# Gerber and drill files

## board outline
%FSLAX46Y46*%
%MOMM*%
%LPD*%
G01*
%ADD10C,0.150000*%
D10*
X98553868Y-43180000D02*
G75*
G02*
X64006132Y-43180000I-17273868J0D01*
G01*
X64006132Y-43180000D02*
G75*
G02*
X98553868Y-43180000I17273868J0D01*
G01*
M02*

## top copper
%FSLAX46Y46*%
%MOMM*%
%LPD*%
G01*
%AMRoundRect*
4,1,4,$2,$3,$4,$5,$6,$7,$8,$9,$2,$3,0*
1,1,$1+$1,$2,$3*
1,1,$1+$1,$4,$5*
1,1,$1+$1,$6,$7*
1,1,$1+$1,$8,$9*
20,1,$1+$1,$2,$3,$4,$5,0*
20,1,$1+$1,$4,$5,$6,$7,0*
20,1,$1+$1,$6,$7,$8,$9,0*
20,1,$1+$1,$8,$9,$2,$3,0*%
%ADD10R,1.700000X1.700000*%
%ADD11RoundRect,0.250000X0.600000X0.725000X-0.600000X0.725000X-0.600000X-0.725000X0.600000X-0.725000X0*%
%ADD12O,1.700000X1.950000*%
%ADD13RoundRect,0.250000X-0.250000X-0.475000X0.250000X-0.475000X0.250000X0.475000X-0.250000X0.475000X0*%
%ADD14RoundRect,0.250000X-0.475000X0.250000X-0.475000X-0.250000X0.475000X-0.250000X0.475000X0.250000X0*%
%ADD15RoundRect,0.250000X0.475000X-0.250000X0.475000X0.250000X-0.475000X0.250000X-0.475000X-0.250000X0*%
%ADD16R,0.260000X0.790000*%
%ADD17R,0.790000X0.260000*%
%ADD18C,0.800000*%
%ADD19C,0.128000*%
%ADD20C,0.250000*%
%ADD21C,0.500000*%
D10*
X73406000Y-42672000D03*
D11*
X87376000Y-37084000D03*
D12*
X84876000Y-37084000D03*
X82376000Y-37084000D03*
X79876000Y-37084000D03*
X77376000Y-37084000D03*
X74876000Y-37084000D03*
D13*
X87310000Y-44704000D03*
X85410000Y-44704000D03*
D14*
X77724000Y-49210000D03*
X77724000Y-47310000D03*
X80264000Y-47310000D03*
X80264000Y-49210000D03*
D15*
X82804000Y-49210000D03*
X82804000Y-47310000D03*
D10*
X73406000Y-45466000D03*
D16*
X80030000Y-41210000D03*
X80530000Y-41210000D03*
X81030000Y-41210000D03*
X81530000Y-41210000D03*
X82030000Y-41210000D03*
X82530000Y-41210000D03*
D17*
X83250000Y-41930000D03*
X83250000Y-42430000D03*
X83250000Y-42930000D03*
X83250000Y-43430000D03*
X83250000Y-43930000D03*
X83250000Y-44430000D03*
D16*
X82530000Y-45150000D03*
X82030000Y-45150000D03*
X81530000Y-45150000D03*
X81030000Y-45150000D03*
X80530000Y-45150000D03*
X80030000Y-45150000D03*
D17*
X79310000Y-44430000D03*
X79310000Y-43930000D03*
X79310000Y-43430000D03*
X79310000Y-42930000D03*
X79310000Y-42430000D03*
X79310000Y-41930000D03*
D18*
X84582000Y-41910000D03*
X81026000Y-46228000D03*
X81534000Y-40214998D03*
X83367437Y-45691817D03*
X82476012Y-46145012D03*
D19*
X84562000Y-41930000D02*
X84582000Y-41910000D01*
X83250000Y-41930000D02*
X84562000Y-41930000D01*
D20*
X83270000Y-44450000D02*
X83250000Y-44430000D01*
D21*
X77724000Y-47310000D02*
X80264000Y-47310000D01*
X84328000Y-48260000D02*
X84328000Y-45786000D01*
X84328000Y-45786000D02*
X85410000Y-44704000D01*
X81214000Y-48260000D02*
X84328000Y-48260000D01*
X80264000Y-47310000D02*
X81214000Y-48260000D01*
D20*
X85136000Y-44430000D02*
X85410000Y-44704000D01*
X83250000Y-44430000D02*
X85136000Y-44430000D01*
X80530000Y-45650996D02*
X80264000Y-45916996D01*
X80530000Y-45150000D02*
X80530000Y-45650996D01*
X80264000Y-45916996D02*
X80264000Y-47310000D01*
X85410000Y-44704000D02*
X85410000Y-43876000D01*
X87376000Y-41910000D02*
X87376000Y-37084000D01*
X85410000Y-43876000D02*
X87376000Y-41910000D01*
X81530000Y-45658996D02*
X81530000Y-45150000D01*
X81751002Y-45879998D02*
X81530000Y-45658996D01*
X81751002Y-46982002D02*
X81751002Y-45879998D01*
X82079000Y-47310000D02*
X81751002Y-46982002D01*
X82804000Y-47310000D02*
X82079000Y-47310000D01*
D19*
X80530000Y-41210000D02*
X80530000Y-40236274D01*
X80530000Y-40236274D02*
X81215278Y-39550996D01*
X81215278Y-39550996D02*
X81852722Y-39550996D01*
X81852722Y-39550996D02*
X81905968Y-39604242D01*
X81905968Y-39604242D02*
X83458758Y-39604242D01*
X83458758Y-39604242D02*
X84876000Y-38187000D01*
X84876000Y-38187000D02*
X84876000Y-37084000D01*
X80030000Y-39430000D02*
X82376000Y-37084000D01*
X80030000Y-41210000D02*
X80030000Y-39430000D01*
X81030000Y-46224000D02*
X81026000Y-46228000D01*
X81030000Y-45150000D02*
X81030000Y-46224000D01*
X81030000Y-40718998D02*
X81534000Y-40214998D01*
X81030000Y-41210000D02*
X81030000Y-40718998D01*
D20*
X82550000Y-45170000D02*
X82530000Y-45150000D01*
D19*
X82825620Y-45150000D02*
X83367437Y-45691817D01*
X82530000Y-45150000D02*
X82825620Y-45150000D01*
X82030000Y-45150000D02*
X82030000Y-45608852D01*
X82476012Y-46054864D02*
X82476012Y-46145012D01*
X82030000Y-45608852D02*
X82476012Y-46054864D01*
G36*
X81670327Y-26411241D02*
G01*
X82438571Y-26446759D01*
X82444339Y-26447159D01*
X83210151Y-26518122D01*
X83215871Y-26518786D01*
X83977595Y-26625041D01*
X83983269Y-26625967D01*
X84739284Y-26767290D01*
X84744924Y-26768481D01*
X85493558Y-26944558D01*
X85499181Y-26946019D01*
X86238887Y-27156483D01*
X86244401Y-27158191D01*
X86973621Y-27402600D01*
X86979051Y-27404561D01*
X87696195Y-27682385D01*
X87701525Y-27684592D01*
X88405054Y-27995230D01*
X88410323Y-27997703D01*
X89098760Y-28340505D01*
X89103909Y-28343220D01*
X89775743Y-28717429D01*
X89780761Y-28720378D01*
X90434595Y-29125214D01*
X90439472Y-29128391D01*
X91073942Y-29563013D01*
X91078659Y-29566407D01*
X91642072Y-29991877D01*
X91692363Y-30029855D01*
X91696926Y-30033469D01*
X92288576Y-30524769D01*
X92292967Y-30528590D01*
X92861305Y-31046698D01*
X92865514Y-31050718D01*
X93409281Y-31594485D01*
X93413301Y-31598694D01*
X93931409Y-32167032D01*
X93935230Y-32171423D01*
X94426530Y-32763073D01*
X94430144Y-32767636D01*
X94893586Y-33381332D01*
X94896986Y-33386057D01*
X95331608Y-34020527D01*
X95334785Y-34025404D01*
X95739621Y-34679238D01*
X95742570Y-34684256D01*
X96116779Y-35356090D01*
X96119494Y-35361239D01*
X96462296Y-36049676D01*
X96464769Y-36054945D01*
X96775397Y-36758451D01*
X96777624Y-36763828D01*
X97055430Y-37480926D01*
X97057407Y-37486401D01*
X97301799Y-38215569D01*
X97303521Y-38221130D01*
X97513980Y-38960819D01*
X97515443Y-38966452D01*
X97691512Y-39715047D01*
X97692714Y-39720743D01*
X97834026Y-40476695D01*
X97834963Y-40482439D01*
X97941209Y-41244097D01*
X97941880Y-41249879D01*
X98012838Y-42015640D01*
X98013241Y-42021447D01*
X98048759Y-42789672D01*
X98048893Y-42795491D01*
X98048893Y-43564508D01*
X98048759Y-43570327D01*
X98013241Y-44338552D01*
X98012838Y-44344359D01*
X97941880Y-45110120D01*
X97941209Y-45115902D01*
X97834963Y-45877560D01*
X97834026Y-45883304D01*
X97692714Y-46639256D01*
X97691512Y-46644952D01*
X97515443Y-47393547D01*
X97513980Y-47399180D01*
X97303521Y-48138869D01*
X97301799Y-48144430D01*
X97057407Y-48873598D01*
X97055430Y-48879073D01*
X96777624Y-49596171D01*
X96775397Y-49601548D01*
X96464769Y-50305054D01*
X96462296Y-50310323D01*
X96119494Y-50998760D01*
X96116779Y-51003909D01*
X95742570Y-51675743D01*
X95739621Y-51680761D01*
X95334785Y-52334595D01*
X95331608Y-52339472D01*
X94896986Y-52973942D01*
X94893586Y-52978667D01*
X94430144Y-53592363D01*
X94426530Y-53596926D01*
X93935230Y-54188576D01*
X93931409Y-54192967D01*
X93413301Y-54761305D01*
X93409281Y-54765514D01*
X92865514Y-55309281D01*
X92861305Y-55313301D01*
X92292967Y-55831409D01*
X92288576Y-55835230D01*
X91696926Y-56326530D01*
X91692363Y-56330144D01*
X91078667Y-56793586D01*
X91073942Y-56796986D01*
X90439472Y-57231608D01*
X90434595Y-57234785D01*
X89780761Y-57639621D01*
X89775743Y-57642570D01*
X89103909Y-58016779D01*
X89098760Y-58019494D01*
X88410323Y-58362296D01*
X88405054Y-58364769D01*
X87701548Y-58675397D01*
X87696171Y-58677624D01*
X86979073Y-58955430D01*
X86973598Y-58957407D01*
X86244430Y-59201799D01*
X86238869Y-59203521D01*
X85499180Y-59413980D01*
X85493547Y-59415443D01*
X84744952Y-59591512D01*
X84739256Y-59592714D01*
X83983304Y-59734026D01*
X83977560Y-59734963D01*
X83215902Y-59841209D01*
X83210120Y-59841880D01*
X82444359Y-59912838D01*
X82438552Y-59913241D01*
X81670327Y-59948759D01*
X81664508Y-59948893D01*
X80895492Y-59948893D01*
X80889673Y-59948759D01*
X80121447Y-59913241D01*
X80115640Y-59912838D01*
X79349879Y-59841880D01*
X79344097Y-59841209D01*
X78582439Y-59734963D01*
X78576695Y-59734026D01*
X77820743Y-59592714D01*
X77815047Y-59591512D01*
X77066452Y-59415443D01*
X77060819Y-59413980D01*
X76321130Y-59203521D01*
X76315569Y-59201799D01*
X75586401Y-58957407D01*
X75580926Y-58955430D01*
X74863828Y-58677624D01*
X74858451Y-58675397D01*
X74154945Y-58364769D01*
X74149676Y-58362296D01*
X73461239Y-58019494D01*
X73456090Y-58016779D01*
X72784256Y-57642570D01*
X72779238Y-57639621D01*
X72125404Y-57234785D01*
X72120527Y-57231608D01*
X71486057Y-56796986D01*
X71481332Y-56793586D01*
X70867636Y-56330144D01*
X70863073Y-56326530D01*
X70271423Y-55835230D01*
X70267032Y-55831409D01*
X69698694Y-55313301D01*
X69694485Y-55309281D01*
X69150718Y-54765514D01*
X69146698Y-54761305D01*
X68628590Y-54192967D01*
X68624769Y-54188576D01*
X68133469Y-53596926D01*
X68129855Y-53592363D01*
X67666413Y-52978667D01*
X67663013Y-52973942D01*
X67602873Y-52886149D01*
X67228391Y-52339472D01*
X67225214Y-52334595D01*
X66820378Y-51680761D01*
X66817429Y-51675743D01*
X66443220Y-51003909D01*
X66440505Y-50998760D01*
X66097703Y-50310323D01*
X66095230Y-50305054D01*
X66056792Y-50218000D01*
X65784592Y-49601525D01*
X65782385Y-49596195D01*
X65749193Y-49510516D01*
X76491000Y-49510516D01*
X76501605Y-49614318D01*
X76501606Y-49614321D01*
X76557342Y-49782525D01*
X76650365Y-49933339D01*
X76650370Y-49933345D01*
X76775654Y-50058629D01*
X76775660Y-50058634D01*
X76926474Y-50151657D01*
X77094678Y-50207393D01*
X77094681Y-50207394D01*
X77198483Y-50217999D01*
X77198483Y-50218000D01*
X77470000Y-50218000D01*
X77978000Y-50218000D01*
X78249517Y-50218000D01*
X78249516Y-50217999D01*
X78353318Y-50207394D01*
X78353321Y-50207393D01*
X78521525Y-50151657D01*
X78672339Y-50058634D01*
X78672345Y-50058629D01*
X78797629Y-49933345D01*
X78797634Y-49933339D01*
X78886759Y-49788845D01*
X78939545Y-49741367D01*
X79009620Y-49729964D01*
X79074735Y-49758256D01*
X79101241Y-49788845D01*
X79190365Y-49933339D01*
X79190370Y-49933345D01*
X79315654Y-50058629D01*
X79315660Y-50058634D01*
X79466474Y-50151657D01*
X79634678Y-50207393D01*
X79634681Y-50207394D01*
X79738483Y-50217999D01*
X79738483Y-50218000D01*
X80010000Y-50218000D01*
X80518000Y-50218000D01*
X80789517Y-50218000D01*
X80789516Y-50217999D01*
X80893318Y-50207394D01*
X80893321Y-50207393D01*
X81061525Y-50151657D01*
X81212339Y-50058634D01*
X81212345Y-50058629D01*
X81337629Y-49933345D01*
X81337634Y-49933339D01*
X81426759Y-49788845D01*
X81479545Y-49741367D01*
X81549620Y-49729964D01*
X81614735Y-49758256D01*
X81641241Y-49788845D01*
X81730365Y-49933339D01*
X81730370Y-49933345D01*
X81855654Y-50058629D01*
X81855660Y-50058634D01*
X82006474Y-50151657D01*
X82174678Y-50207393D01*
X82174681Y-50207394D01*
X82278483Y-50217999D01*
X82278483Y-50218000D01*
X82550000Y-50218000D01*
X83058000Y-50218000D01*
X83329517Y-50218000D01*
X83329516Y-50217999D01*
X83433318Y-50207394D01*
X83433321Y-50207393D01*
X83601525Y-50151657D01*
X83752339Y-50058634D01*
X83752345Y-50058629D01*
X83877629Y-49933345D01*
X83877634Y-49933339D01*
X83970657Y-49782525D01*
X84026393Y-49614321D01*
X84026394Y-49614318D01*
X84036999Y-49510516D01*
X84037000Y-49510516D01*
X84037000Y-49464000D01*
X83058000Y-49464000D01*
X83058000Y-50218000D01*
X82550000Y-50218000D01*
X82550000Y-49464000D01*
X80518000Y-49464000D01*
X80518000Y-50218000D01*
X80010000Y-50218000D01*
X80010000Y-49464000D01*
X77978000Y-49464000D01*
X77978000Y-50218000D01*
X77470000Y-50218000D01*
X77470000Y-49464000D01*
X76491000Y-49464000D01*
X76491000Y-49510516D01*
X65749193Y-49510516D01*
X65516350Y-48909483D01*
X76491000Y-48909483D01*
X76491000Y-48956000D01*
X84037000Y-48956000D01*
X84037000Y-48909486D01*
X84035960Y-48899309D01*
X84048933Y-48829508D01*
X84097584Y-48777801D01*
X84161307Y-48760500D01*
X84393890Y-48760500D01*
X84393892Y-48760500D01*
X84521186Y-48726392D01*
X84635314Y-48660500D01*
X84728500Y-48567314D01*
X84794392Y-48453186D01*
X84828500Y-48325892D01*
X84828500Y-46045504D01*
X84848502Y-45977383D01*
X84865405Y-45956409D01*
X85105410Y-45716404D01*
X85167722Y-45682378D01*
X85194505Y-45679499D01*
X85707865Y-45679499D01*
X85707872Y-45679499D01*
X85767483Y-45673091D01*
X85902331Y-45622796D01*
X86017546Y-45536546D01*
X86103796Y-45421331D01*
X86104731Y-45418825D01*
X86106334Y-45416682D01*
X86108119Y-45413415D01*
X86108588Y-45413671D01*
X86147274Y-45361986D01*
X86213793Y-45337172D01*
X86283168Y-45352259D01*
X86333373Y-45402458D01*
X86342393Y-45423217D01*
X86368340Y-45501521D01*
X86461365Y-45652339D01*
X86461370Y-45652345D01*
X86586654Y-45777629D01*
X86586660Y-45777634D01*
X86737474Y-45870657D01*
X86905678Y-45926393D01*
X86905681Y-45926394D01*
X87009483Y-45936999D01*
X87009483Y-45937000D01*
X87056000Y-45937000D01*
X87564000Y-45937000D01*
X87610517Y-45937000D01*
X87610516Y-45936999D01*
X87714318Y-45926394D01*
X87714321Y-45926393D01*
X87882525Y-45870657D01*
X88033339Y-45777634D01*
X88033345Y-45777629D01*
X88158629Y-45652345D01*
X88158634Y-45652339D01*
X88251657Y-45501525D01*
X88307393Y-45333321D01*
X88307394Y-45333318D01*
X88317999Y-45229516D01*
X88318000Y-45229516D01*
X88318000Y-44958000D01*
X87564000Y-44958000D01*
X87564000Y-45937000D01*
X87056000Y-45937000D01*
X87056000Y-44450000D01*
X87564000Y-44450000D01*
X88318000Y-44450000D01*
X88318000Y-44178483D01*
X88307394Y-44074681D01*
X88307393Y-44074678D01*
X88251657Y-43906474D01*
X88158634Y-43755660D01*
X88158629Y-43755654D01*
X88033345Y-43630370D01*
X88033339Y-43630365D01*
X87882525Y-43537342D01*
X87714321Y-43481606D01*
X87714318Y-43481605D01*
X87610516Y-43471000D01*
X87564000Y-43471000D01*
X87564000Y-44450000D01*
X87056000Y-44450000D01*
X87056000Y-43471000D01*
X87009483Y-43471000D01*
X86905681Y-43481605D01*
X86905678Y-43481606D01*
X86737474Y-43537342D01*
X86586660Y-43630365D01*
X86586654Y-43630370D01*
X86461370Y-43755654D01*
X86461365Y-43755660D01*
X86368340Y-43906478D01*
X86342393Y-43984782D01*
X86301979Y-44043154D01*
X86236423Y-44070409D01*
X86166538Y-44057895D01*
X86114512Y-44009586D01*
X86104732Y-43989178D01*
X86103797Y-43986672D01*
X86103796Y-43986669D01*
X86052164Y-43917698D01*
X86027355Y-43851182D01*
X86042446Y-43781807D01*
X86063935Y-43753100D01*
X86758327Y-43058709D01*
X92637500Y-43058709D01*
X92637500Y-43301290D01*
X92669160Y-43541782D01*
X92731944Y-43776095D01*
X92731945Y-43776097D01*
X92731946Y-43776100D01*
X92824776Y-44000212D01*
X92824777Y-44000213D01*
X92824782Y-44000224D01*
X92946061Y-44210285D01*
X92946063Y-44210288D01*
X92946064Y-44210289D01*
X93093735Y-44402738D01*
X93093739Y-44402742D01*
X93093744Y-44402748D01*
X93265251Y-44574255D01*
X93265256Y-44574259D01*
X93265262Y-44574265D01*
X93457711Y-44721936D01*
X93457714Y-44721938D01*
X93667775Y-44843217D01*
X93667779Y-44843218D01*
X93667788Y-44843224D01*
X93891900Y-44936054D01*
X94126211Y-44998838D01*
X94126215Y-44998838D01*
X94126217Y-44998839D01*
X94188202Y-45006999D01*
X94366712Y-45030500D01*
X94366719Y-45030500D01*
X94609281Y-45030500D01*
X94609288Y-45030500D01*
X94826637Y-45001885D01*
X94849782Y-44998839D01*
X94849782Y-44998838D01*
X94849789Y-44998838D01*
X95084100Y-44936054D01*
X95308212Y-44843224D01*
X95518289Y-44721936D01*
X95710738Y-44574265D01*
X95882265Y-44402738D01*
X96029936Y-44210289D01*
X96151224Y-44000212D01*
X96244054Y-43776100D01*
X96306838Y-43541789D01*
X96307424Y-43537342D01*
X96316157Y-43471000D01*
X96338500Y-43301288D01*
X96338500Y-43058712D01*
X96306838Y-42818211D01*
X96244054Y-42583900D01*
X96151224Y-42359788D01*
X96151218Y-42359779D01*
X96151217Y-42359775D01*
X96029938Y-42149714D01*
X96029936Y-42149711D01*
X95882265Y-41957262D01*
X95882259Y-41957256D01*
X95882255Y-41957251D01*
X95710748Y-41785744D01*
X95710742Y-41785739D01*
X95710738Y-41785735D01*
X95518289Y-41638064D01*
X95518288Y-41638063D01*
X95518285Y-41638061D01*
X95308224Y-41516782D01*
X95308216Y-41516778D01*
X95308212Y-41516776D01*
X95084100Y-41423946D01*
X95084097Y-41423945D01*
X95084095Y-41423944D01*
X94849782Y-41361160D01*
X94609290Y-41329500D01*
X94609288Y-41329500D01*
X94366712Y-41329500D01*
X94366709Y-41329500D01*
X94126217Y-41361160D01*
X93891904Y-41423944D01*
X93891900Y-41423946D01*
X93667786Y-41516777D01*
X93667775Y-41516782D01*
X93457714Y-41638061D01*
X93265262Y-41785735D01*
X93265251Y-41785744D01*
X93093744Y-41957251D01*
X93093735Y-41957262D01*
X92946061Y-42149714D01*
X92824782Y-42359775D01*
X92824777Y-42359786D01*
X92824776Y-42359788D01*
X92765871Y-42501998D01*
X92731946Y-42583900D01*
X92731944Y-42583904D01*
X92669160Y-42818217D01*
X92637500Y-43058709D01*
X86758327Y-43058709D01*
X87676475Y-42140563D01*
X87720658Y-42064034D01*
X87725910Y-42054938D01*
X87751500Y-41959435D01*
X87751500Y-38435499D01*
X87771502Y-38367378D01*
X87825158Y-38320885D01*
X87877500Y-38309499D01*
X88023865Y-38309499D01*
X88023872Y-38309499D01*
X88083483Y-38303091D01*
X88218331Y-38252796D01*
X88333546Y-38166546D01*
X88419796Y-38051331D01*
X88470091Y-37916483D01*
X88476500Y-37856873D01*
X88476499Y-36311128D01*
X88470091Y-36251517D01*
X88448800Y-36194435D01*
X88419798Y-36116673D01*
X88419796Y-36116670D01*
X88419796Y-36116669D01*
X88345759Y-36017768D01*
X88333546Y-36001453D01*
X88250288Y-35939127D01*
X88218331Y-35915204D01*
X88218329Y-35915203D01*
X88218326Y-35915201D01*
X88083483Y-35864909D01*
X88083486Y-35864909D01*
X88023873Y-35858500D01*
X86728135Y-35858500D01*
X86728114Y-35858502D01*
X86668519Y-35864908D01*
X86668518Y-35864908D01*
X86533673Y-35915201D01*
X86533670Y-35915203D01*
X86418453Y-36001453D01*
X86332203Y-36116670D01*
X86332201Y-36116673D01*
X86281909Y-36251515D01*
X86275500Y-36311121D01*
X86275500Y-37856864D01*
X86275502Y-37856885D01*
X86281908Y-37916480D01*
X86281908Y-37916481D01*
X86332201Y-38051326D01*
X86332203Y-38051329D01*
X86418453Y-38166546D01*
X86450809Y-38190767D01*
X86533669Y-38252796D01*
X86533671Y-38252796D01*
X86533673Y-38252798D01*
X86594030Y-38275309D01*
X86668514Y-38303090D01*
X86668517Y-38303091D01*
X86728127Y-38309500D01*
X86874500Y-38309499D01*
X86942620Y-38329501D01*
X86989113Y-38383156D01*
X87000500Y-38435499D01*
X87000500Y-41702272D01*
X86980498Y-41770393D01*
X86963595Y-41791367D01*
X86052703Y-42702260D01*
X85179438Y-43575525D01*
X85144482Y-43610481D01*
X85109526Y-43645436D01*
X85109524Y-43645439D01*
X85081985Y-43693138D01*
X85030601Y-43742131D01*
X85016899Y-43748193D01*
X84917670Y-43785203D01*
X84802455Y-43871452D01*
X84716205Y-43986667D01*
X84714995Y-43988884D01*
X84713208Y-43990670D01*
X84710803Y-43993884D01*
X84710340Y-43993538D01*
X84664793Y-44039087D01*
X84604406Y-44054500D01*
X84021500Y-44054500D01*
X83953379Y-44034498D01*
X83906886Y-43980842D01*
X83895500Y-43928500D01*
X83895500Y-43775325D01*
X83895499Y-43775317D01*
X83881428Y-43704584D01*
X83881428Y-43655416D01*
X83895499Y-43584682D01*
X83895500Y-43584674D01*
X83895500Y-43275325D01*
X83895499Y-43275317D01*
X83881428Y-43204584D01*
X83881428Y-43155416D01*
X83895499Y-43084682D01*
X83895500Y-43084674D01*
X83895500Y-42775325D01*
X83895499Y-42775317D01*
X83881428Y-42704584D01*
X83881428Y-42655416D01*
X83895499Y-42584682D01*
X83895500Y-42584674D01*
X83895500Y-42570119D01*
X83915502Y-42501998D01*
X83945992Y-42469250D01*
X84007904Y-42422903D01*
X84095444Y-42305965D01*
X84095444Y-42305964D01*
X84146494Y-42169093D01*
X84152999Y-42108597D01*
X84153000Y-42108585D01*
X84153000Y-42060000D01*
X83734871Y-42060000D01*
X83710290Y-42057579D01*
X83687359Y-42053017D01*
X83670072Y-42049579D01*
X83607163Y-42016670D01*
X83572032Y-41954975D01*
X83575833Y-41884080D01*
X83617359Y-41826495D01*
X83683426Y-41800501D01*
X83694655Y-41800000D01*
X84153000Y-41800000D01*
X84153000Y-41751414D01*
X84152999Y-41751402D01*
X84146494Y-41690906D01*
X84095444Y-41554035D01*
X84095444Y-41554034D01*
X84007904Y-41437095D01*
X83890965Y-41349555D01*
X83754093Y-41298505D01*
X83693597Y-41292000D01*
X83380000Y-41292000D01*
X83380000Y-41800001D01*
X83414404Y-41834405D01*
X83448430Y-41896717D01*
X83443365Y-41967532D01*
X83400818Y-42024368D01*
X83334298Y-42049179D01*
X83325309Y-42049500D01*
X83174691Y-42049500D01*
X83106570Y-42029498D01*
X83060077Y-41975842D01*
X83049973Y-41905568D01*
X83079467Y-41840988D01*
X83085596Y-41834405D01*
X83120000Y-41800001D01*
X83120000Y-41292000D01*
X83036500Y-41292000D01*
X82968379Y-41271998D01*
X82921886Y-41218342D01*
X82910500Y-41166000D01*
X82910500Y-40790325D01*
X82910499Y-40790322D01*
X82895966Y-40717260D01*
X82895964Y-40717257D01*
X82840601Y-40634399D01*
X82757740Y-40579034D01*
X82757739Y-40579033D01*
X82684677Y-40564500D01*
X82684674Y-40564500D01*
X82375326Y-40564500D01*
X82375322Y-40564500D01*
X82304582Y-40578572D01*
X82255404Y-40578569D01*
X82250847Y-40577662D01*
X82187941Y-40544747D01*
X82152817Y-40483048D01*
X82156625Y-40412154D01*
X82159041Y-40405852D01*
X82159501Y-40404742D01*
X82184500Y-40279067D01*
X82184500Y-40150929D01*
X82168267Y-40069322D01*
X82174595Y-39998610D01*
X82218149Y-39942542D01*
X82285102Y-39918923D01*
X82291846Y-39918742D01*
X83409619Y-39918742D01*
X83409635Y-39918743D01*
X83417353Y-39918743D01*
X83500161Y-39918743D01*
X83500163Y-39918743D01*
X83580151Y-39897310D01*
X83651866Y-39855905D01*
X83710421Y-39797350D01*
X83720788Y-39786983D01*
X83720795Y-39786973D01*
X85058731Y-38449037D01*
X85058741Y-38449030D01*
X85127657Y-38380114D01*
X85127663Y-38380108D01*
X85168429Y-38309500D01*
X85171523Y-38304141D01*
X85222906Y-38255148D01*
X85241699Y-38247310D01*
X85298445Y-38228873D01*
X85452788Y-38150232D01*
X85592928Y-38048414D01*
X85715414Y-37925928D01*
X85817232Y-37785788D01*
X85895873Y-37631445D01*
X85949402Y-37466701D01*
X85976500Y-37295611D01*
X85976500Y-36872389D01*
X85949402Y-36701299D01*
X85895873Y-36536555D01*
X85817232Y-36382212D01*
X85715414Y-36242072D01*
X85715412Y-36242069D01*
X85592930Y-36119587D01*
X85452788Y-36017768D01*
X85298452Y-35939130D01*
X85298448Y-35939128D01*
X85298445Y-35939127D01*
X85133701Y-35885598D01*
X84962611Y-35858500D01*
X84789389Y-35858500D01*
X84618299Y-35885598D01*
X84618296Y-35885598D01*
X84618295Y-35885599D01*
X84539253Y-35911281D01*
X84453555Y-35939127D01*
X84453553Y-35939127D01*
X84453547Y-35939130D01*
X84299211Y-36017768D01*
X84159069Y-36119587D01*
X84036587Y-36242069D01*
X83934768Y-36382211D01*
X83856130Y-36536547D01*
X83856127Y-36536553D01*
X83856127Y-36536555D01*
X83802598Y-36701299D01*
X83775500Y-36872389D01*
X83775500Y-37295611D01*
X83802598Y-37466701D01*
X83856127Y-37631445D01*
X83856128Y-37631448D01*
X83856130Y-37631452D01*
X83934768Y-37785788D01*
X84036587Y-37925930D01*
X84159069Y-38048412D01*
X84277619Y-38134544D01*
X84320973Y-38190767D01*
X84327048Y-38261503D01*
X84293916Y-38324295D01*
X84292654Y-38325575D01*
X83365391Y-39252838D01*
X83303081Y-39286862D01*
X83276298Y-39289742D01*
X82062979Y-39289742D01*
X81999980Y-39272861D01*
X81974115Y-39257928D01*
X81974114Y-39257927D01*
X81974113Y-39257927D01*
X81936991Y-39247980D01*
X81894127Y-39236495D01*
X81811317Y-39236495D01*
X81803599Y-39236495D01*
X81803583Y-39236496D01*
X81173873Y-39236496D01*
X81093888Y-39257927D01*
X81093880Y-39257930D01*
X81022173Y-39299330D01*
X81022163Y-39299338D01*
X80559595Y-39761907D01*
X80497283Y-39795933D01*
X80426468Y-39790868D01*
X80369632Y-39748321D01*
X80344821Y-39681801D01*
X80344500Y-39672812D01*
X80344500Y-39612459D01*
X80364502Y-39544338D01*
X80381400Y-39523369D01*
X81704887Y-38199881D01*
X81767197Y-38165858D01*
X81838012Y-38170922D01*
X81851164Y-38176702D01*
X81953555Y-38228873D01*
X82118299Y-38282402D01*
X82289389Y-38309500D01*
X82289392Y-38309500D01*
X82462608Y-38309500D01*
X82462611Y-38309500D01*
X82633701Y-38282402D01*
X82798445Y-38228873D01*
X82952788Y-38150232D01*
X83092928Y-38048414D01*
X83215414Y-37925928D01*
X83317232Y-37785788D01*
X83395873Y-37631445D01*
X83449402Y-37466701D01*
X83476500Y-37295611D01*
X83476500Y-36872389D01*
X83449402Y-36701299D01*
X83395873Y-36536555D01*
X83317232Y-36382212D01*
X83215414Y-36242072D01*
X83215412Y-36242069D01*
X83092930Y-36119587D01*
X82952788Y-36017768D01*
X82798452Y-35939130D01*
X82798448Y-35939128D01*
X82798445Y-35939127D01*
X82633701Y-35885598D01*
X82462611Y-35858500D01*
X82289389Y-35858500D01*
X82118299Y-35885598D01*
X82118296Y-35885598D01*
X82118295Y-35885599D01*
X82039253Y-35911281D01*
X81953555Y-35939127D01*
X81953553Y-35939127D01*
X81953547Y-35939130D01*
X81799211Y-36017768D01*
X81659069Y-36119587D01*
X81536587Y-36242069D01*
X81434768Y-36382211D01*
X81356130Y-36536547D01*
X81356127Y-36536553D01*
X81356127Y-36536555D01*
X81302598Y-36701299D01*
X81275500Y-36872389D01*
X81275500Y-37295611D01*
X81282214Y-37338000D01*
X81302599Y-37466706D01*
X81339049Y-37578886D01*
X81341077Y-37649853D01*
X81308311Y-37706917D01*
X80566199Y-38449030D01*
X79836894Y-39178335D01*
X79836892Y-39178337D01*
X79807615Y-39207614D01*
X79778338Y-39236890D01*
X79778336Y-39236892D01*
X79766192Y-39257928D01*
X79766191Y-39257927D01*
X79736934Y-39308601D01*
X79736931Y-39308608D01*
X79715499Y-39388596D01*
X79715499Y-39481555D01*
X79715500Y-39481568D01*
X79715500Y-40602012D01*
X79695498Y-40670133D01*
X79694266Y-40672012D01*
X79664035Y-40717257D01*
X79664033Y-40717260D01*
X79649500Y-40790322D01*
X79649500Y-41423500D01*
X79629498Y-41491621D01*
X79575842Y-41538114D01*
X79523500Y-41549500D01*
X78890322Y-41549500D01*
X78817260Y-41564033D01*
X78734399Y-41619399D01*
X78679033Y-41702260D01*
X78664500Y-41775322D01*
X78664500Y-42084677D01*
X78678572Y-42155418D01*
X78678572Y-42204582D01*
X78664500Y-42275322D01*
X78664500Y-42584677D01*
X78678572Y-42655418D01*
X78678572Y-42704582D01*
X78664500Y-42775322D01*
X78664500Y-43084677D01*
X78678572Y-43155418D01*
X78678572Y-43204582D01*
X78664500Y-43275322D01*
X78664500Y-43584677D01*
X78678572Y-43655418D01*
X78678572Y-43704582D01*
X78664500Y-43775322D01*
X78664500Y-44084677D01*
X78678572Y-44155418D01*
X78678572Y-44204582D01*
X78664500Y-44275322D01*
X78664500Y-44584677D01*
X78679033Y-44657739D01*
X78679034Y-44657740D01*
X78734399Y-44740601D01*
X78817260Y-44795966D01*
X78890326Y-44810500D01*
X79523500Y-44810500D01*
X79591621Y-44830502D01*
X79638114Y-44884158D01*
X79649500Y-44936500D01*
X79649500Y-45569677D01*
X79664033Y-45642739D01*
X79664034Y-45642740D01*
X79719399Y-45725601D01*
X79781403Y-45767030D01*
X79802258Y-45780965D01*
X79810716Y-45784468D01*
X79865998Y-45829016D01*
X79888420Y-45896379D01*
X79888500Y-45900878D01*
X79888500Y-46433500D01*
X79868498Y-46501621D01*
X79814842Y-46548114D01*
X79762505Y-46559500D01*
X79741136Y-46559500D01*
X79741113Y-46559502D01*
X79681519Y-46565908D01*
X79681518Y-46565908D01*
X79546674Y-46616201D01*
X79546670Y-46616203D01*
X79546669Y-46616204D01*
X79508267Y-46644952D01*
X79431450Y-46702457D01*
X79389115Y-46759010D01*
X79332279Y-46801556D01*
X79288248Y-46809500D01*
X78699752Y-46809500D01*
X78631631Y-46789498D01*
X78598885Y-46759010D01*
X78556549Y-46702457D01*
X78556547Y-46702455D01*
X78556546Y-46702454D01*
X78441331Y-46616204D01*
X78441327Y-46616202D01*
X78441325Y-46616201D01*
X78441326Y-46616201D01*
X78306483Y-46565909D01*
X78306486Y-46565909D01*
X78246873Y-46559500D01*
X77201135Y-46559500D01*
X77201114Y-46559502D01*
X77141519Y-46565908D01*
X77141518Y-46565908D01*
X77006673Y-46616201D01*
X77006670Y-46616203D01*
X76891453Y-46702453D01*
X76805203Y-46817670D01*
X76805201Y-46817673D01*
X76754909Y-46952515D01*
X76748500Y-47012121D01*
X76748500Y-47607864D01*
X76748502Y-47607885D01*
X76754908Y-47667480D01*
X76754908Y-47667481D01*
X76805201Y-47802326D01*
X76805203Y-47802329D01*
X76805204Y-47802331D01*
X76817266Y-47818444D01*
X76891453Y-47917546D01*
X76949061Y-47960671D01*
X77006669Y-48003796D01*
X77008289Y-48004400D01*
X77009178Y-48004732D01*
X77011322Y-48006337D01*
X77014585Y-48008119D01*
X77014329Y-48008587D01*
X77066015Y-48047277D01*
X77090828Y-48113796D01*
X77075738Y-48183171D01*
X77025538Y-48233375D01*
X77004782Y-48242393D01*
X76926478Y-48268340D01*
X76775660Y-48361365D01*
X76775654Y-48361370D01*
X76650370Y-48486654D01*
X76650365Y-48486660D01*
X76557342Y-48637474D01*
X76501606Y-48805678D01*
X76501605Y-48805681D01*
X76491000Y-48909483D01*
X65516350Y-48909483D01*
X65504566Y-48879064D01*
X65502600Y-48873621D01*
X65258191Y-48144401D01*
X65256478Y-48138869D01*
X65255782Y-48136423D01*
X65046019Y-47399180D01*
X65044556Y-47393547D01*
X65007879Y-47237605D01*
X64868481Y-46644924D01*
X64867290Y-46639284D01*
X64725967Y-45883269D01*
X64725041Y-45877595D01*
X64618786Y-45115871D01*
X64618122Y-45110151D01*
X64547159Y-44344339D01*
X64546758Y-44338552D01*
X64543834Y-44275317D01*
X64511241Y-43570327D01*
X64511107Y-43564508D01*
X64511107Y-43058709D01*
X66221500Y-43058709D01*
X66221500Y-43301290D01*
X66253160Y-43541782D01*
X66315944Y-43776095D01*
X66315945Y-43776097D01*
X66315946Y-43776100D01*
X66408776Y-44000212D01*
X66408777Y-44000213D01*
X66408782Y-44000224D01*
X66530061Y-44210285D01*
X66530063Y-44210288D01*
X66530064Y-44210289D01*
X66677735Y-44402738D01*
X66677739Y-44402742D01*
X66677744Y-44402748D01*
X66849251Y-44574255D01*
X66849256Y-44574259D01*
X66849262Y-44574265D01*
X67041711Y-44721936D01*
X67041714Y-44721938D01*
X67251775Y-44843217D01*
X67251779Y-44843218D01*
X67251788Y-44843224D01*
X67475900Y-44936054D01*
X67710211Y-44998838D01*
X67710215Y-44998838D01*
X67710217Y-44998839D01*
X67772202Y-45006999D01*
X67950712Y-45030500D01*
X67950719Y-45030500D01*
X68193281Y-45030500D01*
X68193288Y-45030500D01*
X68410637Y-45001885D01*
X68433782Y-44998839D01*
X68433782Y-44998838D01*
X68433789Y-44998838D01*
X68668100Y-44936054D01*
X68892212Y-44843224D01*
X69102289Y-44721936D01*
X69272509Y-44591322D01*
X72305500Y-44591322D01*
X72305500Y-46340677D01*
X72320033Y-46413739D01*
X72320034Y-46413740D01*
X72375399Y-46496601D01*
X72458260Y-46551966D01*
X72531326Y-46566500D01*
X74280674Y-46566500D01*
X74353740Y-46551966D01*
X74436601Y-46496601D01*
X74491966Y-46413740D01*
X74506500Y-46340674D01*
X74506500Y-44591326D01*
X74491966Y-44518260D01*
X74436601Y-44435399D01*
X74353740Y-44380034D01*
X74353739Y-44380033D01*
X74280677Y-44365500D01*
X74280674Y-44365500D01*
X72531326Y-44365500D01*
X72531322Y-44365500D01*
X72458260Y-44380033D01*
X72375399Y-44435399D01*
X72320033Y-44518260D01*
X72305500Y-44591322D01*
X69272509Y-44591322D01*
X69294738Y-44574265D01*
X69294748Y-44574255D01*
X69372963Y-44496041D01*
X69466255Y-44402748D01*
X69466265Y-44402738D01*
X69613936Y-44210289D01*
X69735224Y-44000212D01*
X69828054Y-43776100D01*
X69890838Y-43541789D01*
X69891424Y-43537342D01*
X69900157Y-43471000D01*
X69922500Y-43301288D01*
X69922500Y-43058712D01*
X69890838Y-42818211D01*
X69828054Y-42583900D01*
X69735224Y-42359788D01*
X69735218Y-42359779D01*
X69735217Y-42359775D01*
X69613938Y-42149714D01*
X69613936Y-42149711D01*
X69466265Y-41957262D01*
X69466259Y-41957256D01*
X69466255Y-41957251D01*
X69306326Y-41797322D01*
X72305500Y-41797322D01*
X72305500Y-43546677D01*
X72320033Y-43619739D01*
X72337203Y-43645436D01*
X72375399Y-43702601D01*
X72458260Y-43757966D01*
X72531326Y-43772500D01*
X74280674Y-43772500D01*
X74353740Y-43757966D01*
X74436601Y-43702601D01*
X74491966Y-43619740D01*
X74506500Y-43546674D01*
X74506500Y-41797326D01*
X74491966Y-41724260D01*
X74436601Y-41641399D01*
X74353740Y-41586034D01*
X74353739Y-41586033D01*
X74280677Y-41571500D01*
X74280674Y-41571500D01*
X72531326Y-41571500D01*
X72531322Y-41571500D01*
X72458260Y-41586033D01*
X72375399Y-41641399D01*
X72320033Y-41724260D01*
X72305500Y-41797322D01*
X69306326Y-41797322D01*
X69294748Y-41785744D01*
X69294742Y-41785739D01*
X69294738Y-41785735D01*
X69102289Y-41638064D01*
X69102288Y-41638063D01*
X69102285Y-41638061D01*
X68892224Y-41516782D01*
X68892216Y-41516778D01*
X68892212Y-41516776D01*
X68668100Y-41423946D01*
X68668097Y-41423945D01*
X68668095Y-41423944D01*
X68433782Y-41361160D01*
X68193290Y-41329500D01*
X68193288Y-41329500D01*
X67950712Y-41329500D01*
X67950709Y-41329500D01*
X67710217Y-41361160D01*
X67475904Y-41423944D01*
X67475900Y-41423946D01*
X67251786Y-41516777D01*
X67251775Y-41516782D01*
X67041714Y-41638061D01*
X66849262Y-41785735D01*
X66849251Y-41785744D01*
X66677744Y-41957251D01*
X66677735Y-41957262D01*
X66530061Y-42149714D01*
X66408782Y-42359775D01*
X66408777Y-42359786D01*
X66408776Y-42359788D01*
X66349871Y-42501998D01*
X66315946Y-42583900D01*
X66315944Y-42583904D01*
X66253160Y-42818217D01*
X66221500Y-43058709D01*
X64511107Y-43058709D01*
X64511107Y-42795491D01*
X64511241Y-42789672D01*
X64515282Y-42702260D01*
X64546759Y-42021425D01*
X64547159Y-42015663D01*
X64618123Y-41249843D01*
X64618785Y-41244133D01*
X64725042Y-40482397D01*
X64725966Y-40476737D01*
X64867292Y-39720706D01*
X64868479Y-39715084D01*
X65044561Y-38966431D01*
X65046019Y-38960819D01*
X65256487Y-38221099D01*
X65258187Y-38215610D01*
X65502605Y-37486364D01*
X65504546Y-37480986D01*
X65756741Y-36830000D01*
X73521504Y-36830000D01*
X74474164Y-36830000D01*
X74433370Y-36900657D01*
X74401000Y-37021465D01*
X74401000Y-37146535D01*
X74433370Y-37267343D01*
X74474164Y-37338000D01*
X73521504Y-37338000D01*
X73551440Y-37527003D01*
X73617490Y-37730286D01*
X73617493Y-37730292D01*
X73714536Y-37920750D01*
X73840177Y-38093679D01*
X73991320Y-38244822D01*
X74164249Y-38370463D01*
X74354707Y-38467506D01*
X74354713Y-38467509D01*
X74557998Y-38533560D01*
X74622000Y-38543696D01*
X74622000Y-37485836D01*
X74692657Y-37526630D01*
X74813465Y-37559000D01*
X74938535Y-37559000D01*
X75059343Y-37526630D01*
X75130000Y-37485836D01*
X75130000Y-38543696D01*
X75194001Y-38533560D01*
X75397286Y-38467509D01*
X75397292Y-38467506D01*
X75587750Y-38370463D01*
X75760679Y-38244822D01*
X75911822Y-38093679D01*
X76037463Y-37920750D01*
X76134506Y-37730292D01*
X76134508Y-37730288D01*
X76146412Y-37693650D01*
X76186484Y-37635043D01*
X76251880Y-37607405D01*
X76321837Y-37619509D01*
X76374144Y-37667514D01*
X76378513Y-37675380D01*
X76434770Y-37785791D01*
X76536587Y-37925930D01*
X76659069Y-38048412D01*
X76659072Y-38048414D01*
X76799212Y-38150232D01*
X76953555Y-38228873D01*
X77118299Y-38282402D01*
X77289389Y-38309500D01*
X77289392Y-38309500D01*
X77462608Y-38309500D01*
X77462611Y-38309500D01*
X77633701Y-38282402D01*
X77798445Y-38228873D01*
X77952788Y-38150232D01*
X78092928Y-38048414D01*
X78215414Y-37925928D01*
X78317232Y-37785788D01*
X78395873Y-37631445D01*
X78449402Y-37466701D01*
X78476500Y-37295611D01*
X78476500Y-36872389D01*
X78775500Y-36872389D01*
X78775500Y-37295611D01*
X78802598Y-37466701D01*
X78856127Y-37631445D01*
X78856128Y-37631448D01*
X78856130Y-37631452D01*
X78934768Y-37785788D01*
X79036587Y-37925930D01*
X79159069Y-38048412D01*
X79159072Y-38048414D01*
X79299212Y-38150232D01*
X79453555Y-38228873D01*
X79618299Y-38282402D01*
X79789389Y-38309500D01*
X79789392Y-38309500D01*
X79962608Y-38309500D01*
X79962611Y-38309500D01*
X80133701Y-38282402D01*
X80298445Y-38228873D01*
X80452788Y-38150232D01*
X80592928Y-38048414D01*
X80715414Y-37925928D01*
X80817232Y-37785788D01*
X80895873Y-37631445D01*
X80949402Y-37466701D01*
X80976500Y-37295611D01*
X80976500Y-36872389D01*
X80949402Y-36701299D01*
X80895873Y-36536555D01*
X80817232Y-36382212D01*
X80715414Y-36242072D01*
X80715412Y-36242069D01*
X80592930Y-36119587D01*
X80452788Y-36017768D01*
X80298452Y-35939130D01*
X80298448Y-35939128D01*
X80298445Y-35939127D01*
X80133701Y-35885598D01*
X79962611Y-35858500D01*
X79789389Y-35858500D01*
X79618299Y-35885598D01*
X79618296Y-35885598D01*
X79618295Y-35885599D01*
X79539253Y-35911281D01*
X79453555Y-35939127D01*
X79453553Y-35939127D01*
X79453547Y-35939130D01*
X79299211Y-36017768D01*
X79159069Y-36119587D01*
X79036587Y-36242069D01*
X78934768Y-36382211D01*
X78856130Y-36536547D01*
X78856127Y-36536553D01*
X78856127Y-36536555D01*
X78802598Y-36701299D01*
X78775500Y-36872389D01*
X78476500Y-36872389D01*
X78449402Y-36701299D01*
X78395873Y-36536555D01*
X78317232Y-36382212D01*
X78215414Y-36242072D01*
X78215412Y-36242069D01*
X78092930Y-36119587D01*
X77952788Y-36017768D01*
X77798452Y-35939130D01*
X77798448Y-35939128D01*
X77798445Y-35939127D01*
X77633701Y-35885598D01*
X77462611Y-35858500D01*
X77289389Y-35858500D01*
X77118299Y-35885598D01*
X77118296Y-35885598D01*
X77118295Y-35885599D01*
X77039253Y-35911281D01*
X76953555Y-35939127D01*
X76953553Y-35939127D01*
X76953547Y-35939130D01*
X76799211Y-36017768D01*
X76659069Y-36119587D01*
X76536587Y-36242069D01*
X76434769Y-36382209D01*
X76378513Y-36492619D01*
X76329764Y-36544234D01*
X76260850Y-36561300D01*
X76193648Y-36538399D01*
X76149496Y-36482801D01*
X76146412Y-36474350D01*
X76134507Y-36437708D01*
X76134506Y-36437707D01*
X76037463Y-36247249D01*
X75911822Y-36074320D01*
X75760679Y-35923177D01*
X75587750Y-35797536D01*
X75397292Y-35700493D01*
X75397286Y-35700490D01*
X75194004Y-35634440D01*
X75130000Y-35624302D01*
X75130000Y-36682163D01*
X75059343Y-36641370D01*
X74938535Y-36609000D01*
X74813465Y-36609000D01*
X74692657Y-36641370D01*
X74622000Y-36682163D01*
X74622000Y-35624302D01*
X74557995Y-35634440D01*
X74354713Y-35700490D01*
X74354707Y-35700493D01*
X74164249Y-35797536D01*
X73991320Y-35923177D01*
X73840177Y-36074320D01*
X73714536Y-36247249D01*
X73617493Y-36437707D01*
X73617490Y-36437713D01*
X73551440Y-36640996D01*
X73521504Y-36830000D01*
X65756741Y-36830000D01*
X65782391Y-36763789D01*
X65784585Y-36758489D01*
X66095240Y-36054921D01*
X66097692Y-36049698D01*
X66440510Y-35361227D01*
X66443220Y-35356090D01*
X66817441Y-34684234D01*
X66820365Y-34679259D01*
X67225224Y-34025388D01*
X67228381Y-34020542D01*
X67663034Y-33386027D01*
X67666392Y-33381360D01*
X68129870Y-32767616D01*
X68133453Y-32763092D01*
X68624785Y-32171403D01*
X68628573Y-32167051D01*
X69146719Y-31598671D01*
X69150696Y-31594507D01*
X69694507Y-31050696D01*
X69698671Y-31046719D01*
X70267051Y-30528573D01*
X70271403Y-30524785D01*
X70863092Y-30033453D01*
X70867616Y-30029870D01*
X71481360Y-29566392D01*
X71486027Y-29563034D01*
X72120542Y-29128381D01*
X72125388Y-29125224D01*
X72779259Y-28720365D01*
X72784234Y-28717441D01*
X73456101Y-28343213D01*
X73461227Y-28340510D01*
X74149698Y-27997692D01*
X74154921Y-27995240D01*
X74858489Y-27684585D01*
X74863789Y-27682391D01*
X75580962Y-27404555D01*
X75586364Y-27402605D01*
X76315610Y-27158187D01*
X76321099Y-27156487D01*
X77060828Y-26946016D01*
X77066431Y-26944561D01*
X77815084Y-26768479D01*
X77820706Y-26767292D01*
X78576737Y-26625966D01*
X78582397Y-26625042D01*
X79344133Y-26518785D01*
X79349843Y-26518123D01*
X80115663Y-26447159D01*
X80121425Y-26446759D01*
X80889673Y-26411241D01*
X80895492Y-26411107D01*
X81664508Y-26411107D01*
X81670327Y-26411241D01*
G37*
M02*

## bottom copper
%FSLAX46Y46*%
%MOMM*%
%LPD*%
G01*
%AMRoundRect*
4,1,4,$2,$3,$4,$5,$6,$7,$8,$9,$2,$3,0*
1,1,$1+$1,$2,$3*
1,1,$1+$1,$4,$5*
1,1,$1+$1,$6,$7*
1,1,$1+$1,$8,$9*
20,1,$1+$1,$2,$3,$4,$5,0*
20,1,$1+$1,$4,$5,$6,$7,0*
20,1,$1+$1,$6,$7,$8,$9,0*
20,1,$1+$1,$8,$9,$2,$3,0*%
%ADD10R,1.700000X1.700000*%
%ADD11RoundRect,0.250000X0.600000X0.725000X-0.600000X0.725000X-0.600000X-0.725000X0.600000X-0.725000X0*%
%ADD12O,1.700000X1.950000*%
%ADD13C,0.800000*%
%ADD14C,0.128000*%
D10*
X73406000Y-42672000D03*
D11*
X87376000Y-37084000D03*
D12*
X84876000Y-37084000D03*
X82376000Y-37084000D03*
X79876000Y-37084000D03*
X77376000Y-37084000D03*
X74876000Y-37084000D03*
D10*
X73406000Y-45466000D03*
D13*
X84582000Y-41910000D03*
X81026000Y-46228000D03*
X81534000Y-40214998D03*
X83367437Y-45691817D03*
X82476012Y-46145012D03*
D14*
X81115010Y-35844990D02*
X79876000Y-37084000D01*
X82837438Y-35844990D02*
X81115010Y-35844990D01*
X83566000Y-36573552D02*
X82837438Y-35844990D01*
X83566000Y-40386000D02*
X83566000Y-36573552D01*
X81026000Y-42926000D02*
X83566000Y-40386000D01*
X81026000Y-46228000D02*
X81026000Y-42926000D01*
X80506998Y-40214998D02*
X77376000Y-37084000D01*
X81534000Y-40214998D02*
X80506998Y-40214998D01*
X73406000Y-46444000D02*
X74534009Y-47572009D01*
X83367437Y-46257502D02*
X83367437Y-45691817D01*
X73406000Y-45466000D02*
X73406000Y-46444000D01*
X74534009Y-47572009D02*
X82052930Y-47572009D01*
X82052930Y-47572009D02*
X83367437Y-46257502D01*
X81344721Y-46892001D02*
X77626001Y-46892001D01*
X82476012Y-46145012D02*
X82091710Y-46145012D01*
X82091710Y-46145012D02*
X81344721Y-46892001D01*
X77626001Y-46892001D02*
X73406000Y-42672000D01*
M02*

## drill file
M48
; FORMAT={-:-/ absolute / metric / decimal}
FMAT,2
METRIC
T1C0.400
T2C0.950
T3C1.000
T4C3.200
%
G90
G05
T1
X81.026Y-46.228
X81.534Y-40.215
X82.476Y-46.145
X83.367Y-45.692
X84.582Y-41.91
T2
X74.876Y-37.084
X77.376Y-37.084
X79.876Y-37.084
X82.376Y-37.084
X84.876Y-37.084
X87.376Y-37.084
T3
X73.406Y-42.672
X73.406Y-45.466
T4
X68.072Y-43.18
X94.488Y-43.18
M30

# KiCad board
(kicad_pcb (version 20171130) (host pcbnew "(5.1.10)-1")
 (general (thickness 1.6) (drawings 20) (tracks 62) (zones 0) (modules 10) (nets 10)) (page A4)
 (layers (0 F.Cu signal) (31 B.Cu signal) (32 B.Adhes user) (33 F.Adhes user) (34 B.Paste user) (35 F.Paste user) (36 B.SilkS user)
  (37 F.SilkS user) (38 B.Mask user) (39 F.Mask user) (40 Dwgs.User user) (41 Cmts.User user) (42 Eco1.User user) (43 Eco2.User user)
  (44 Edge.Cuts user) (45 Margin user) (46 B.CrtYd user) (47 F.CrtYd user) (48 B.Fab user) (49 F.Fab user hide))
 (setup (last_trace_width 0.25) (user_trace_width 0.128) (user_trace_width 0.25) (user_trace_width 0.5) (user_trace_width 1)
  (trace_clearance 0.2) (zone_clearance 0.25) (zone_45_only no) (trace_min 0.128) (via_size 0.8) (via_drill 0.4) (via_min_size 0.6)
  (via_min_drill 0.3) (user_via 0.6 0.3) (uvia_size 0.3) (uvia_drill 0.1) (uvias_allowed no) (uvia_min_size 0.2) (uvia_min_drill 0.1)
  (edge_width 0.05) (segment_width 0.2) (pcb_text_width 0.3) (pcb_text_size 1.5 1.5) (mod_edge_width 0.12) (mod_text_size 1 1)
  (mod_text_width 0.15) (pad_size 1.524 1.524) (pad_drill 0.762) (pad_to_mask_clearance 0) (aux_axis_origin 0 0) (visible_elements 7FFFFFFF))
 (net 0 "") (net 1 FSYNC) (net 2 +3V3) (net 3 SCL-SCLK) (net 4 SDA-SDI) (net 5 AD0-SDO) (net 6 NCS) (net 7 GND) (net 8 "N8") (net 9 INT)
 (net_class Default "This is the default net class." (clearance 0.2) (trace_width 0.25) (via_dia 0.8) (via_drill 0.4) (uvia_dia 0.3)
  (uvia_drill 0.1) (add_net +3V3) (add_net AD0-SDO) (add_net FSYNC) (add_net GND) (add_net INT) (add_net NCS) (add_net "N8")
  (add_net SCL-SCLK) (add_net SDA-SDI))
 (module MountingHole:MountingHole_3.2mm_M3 (layer F.Cu) (at 94.488 43.18)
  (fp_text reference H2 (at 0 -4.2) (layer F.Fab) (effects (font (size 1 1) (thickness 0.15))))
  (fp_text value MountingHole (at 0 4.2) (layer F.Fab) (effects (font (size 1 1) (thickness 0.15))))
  (pad 1 np_thru_hole circle (at 0 0) (size 3.2 3.2) (drill 3.2) (layers *.Cu *.Mask)))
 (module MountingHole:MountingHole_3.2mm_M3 (layer F.Cu) (at 68.072 43.18)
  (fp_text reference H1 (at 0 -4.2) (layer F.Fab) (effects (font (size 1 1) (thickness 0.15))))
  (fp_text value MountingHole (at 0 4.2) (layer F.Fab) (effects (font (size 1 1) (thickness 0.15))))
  (pad 1 np_thru_hole circle (at 0 0) (size 3.2 3.2) (drill 3.2) (layers *.Cu *.Mask)))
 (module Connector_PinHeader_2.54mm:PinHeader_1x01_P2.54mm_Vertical (layer F.Cu) (at 73.406 42.672)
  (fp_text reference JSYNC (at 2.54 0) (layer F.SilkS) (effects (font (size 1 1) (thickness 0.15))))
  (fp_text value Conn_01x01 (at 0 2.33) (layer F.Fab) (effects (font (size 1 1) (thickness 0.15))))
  (pad 1 thru_hole rect (at 0 0) (size 1.7 1.7) (drill 1) (layers *.Cu *.Mask) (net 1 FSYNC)))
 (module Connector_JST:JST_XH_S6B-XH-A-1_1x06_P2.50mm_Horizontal (layer F.Cu) (at 87.376 37.084 180)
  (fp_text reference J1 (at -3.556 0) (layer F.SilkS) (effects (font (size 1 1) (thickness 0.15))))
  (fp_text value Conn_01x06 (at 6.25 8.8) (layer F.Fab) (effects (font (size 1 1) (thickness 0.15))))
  (pad 1 thru_hole roundrect (at 0 0 180) (size 1.7 1.95) (drill 0.95) (layers *.Cu *.Mask) (roundrect_rratio 0.1470588235294118)
   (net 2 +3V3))
  (pad 2 thru_hole oval (at 2.5 0 180) (size 1.7 1.95) (drill 0.95) (layers *.Cu *.Mask) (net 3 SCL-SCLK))
  (pad 3 thru_hole oval (at 5 0 180) (size 1.7 1.95) (drill 0.95) (layers *.Cu *.Mask) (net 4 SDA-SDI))
  (pad 4 thru_hole oval (at 7.5 0 180) (size 1.7 1.95) (drill 0.95) (layers *.Cu *.Mask) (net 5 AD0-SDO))
  (pad 5 thru_hole oval (at 10 0 180) (size 1.7 1.95) (drill 0.95) (layers *.Cu *.Mask) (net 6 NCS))
  (pad 6 thru_hole oval (at 12.5 0 180) (size 1.7 1.95) (drill 0.95) (layers *.Cu *.Mask) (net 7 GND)))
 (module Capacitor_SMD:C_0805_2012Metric (layer F.Cu) (at 86.36 44.704)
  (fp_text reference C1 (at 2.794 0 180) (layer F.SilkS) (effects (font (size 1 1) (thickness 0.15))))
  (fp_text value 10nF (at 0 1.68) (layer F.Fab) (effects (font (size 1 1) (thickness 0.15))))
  (pad 2 smd roundrect (at 0.95 0) (size 1 1.45) (layers F.Cu F.Paste F.Mask) (roundrect_rratio 0.25) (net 7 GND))
  (pad 1 smd roundrect (at -0.95 0) (size 1 1.45) (layers F.Cu F.Paste F.Mask) (roundrect_rratio 0.25) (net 2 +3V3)))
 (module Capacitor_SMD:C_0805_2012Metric (layer F.Cu) (at 77.724 48.26 270)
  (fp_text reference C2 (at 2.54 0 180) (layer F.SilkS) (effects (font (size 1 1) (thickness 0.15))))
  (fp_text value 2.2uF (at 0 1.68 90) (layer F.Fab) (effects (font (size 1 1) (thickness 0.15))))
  (pad 2 smd roundrect (at 0.95 0 270) (size 1 1.45) (layers F.Cu F.Paste F.Mask) (roundrect_rratio 0.25) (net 7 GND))
  (pad 1 smd roundrect (at -0.95 0 270) (size 1 1.45) (layers F.Cu F.Paste F.Mask) (roundrect_rratio 0.25) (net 2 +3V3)))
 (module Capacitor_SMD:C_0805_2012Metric (layer F.Cu) (at 80.264 48.26 270)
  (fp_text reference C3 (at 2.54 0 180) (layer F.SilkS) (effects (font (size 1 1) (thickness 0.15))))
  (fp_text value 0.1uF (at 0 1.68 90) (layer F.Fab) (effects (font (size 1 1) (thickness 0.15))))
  (pad 1 smd roundrect (at -0.95 0 270) (size 1 1.45) (layers F.Cu F.Paste F.Mask) (roundrect_rratio 0.25) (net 2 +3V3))
  (pad 2 smd roundrect (at 0.95 0 270) (size 1 1.45) (layers F.Cu F.Paste F.Mask) (roundrect_rratio 0.25) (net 7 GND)))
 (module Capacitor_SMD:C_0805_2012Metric (layer F.Cu) (at 82.804 48.26 90)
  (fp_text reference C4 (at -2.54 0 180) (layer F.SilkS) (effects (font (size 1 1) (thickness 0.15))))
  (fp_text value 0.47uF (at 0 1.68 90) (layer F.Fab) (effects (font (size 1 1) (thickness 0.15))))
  (pad 1 smd roundrect (at -0.95 0 90) (size 1 1.45) (layers F.Cu F.Paste F.Mask) (roundrect_rratio 0.25) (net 7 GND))
  (pad 2 smd roundrect (at 0.95 0 90) (size 1 1.45) (layers F.Cu F.Paste F.Mask) (roundrect_rratio 0.25) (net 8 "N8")))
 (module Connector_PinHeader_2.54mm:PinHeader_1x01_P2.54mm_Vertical (layer F.Cu) (at 73.406 45.466)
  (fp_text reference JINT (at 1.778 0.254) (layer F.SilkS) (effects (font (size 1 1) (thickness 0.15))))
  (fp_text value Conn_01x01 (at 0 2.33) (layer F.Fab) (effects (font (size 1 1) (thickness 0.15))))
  (pad 1 thru_hole rect (at 0 0) (size 1.7 1.7) (drill 1) (layers *.Cu *.Mask) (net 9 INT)))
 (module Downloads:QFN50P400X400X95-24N (layer F.Cu) (at 81.28 43.18)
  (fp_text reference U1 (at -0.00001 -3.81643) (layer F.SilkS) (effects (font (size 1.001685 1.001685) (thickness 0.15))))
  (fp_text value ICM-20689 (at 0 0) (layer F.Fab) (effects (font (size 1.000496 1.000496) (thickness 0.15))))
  (pad 24 smd rect (at -1.25 -1.97) (size 0.26 0.79) (layers F.Cu F.Paste F.Mask) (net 4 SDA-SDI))
  (pad 23 smd rect (at -0.75 -1.97) (size 0.26 0.79) (layers F.Cu F.Paste F.Mask) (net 3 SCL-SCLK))
  (pad 22 smd rect (at -0.25 -1.97) (size 0.26 0.79) (layers F.Cu F.Paste F.Mask) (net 6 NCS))
  (pad 21 smd rect (at 0.25 -1.97) (size 0.26 0.79) (layers F.Cu F.Paste F.Mask))
  (pad 20 smd rect (at 0.75 -1.97) (size 0.26 0.79) (layers F.Cu F.Paste F.Mask))
  (pad 19 smd rect (at 1.25 -1.97) (size 0.26 0.79) (layers F.Cu F.Paste F.Mask))
  (pad 18 smd rect (at 1.97 -1.25) (size 0.79 0.26) (layers F.Cu F.Paste F.Mask) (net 7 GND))
  (pad 17 smd rect (at 1.97 -0.75) (size 0.79 0.26) (layers F.Cu F.Paste F.Mask))
  (pad 16 smd rect (at 1.97 -0.25) (size 0.79 0.26) (layers F.Cu F.Paste F.Mask))
  (pad 15 smd rect (at 1.97 0.25) (size 0.79 0.26) (layers F.Cu F.Paste F.Mask))
  (pad 14 smd rect (at 1.97 0.75) (size 0.79 0.26) (layers F.Cu F.Paste F.Mask))
  (pad 13 smd rect (at 1.97 1.25) (size 0.79 0.26) (layers F.Cu F.Paste F.Mask) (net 2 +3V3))
  (pad 12 smd rect (at 1.25 1.97) (size 0.26 0.79) (layers F.Cu F.Paste F.Mask) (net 9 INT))
  (pad 11 smd rect (at 0.75 1.97) (size 0.26 0.79) (layers F.Cu F.Paste F.Mask) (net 1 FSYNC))
  (pad 10 smd rect (at 0.25 1.97) (size 0.26 0.79) (layers F.Cu F.Paste F.Mask) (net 8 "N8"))
  (pad 9 smd rect (at -0.25 1.97) (size 0.26 0.79) (layers F.Cu F.Paste F.Mask) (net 5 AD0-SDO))
  (pad 8 smd rect (at -0.75 1.97) (size 0.26 0.79) (layers F.Cu F.Paste F.Mask) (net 2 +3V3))
  (pad 7 smd rect (at -1.25 1.97) (size 0.26 0.79) (layers F.Cu F.Paste F.Mask))
  (pad 6 smd rect (at -1.97 1.25) (size 0.79 0.26) (layers F.Cu F.Paste F.Mask))
  (pad 5 smd rect (at -1.97 0.75) (size 0.79 0.26) (layers F.Cu F.Paste F.Mask))
  (pad 4 smd rect (at -1.97 0.25) (size 0.79 0.26) (layers F.Cu F.Paste F.Mask))
  (pad 3 smd rect (at -1.97 -0.25) (size 0.79 0.26) (layers F.Cu F.Paste F.Mask))
  (pad 2 smd rect (at -1.97 -0.75) (size 0.79 0.26) (layers F.Cu F.Paste F.Mask))
  (pad 1 smd rect (at -1.97 -1.25) (size 0.79 0.26) (layers F.Cu F.Paste F.Mask)))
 (gr_circle (center 81.28 43.18) (end 98.552 42.926) (layer Edge.Cuts) (width 0.15))
 (via (at 84.582 41.91) (size 0.8) (drill 0.4) (layers F.Cu B.Cu) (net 7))
 (segment (start 84.562 41.93) (end 84.582 41.91) (width 0.128) (layer F.Cu) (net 7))
 (segment (start 83.25 41.93) (end 84.562 41.93) (width 0.128) (layer F.Cu) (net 7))
 (segment (start 83.27 44.45) (end 83.25 44.43) (width 0.25) (layer F.Cu) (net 2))
 (segment (start 77.724 47.31) (end 80.264 47.31) (width 0.5) (layer F.Cu) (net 2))
 (segment (start 84.328 48.26) (end 84.328 45.786) (width 0.5) (layer F.Cu) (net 2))
 (segment (start 84.328 45.786) (end 85.41 44.704) (width 0.5) (layer F.Cu) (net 2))
 (segment (start 81.214 48.26) (end 84.328 48.26) (width 0.5) (layer F.Cu) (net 2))
 (segment (start 80.264 47.31) (end 81.214 48.26) (width 0.5) (layer F.Cu) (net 2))
 (segment (start 85.136 44.43) (end 85.41 44.704) (width 0.25) (layer F.Cu) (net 2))
 (segment (start 83.25 44.43) (end 85.136 44.43) (width 0.25) (layer F.Cu) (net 2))
 (segment (start 80.53 45.650996) (end 80.264 45.916996) (width 0.25) (layer F.Cu) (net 2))
 (segment (start 80.53 45.15) (end 80.53 45.650996) (width 0.25) (layer F.Cu) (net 2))
 (segment (start 80.264 45.916996) (end 80.264 47.31) (width 0.25) (layer F.Cu) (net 2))
 (segment (start 85.41 44.704) (end 85.41 43.876) (width 0.25) (layer F.Cu) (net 2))
 (segment (start 87.376 41.91) (end 87.376 37.084) (width 0.25) (layer F.Cu) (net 2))
 (segment (start 85.41 43.876) (end 87.376 41.91) (width 0.25) (layer F.Cu) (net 2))
 (segment (start 81.53 45.658996) (end 81.53 45.15) (width 0.25) (layer F.Cu) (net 8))
 (segment (start 81.751002 45.879998) (end 81.53 45.658996) (width 0.25) (layer F.Cu) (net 8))
 (segment (start 81.751002 46.982002) (end 81.751002 45.879998) (width 0.25) (layer F.Cu) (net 8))
 (segment (start 82.079 47.31) (end 81.751002 46.982002) (width 0.25) (layer F.Cu) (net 8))
 (segment (start 82.804 47.31) (end 82.079 47.31) (width 0.25) (layer F.Cu) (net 8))
 (segment (start 80.53 41.21) (end 80.53 40.236274) (width 0.128) (layer F.Cu) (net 3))
 (segment (start 80.53 40.236274) (end 81.215278 39.550996) (width 0.128) (layer F.Cu) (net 3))
 (segment (start 81.215278 39.550996) (end 81.852722 39.550996) (width 0.128) (layer F.Cu) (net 3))
 (segment (start 81.852722 39.550996) (end 81.905968 39.604242) (width 0.128) (layer F.Cu) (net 3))
 (segment (start 81.905968 39.604242) (end 83.458758 39.604242) (width 0.128) (layer F.Cu) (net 3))
 (segment (start 83.458758 39.604242) (end 84.876 38.187) (width 0.128) (layer F.Cu) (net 3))
 (segment (start 84.876 38.187) (end 84.876 37.084) (width 0.128) (layer F.Cu) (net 3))
 (segment (start 80.03 39.43) (end 82.376 37.084) (width 0.128) (layer F.Cu) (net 4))
 (segment (start 80.03 41.21) (end 80.03 39.43) (width 0.128) (layer F.Cu) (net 4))
 (via (at 81.026 46.228) (size 0.8) (drill 0.4) (layers F.Cu B.Cu) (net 5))
 (segment (start 81.03 46.224) (end 81.026 46.228) (width 0.128) (layer F.Cu) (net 5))
 (segment (start 81.03 45.15) (end 81.03 46.224) (width 0.128) (layer F.Cu) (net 5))
 (segment (start 81.11501 35.84499) (end 79.876 37.084) (width 0.128) (layer B.Cu) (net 5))
 (segment (start 82.837438 35.84499) (end 81.11501 35.84499) (width 0.128) (layer B.Cu) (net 5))
 (segment (start 83.566 36.573552) (end 82.837438 35.84499) (width 0.128) (layer B.Cu) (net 5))
 (segment (start 83.566 40.386) (end 83.566 36.573552) (width 0.128) (layer B.Cu) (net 5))
 (segment (start 81.026 42.926) (end 83.566 40.386) (width 0.128) (layer B.Cu) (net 5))
 (segment (start 81.026 46.228) (end 81.026 42.926) (width 0.128) (layer B.Cu) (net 5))
 (via (at 81.534 40.214998) (size 0.8) (drill 0.4) (layers F.Cu B.Cu) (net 6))
 (segment (start 81.03 40.718998) (end 81.534 40.214998) (width 0.128) (layer F.Cu) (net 6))
 (segment (start 81.03 41.21) (end 81.03 40.718998) (width 0.128) (layer F.Cu) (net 6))
 (segment (start 80.506998 40.214998) (end 77.376 37.084) (width 0.128) (layer B.Cu) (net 6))
 (segment (start 81.534 40.214998) (end 80.506998 40.214998) (width 0.128) (layer B.Cu) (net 6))
 (segment (start 82.55 45.17) (end 82.53 45.15) (width 0.25) (layer F.Cu) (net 9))
 (via (at 83.367437 45.691817) (size 0.8) (drill 0.4) (layers F.Cu B.Cu) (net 9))
 (segment (start 82.82562 45.15) (end 83.367437 45.691817) (width 0.128) (layer F.Cu) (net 9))
 (segment (start 82.53 45.15) (end 82.82562 45.15) (width 0.128) (layer F.Cu) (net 9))
 (segment (start 73.406 46.444) (end 74.534009 47.572009) (width 0.128) (layer B.Cu) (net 9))
 (segment (start 83.367437 46.257502) (end 83.367437 45.691817) (width 0.128) (layer B.Cu) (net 9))
 (segment (start 73.406 45.466) (end 73.406 46.444) (width 0.128) (layer B.Cu) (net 9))
 (segment (start 74.534009 47.572009) (end 82.05293 47.572009) (width 0.128) (layer B.Cu) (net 9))
 (segment (start 82.05293 47.572009) (end 83.367437 46.257502) (width 0.128) (layer B.Cu) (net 9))
 (via (at 82.476012 46.145012) (size 0.8) (drill 0.4) (layers F.Cu B.Cu) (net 1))
 (segment (start 82.03 45.15) (end 82.03 45.608852) (width 0.128) (layer F.Cu) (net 1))
 (segment (start 82.476012 46.054864) (end 82.476012 46.145012) (width 0.128) (layer F.Cu) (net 1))
 (segment (start 82.03 45.608852) (end 82.476012 46.054864) (width 0.128) (layer F.Cu) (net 1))
 (segment (start 81.344721 46.892001) (end 77.626001 46.892001) (width 0.128) (layer B.Cu) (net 1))
 (segment (start 82.476012 46.145012) (end 82.09171 46.145012) (width 0.128) (layer B.Cu) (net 1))
 (segment (start 82.09171 46.145012) (end 81.344721 46.892001) (width 0.128) (layer B.Cu) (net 1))
 (segment (start 77.626001 46.892001) (end 73.406 42.672) (width 0.128) (layer B.Cu) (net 1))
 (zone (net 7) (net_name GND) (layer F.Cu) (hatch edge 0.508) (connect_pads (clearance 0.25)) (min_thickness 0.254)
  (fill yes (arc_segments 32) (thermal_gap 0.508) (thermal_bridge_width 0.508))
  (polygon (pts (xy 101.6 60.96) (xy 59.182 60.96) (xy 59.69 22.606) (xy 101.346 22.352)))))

